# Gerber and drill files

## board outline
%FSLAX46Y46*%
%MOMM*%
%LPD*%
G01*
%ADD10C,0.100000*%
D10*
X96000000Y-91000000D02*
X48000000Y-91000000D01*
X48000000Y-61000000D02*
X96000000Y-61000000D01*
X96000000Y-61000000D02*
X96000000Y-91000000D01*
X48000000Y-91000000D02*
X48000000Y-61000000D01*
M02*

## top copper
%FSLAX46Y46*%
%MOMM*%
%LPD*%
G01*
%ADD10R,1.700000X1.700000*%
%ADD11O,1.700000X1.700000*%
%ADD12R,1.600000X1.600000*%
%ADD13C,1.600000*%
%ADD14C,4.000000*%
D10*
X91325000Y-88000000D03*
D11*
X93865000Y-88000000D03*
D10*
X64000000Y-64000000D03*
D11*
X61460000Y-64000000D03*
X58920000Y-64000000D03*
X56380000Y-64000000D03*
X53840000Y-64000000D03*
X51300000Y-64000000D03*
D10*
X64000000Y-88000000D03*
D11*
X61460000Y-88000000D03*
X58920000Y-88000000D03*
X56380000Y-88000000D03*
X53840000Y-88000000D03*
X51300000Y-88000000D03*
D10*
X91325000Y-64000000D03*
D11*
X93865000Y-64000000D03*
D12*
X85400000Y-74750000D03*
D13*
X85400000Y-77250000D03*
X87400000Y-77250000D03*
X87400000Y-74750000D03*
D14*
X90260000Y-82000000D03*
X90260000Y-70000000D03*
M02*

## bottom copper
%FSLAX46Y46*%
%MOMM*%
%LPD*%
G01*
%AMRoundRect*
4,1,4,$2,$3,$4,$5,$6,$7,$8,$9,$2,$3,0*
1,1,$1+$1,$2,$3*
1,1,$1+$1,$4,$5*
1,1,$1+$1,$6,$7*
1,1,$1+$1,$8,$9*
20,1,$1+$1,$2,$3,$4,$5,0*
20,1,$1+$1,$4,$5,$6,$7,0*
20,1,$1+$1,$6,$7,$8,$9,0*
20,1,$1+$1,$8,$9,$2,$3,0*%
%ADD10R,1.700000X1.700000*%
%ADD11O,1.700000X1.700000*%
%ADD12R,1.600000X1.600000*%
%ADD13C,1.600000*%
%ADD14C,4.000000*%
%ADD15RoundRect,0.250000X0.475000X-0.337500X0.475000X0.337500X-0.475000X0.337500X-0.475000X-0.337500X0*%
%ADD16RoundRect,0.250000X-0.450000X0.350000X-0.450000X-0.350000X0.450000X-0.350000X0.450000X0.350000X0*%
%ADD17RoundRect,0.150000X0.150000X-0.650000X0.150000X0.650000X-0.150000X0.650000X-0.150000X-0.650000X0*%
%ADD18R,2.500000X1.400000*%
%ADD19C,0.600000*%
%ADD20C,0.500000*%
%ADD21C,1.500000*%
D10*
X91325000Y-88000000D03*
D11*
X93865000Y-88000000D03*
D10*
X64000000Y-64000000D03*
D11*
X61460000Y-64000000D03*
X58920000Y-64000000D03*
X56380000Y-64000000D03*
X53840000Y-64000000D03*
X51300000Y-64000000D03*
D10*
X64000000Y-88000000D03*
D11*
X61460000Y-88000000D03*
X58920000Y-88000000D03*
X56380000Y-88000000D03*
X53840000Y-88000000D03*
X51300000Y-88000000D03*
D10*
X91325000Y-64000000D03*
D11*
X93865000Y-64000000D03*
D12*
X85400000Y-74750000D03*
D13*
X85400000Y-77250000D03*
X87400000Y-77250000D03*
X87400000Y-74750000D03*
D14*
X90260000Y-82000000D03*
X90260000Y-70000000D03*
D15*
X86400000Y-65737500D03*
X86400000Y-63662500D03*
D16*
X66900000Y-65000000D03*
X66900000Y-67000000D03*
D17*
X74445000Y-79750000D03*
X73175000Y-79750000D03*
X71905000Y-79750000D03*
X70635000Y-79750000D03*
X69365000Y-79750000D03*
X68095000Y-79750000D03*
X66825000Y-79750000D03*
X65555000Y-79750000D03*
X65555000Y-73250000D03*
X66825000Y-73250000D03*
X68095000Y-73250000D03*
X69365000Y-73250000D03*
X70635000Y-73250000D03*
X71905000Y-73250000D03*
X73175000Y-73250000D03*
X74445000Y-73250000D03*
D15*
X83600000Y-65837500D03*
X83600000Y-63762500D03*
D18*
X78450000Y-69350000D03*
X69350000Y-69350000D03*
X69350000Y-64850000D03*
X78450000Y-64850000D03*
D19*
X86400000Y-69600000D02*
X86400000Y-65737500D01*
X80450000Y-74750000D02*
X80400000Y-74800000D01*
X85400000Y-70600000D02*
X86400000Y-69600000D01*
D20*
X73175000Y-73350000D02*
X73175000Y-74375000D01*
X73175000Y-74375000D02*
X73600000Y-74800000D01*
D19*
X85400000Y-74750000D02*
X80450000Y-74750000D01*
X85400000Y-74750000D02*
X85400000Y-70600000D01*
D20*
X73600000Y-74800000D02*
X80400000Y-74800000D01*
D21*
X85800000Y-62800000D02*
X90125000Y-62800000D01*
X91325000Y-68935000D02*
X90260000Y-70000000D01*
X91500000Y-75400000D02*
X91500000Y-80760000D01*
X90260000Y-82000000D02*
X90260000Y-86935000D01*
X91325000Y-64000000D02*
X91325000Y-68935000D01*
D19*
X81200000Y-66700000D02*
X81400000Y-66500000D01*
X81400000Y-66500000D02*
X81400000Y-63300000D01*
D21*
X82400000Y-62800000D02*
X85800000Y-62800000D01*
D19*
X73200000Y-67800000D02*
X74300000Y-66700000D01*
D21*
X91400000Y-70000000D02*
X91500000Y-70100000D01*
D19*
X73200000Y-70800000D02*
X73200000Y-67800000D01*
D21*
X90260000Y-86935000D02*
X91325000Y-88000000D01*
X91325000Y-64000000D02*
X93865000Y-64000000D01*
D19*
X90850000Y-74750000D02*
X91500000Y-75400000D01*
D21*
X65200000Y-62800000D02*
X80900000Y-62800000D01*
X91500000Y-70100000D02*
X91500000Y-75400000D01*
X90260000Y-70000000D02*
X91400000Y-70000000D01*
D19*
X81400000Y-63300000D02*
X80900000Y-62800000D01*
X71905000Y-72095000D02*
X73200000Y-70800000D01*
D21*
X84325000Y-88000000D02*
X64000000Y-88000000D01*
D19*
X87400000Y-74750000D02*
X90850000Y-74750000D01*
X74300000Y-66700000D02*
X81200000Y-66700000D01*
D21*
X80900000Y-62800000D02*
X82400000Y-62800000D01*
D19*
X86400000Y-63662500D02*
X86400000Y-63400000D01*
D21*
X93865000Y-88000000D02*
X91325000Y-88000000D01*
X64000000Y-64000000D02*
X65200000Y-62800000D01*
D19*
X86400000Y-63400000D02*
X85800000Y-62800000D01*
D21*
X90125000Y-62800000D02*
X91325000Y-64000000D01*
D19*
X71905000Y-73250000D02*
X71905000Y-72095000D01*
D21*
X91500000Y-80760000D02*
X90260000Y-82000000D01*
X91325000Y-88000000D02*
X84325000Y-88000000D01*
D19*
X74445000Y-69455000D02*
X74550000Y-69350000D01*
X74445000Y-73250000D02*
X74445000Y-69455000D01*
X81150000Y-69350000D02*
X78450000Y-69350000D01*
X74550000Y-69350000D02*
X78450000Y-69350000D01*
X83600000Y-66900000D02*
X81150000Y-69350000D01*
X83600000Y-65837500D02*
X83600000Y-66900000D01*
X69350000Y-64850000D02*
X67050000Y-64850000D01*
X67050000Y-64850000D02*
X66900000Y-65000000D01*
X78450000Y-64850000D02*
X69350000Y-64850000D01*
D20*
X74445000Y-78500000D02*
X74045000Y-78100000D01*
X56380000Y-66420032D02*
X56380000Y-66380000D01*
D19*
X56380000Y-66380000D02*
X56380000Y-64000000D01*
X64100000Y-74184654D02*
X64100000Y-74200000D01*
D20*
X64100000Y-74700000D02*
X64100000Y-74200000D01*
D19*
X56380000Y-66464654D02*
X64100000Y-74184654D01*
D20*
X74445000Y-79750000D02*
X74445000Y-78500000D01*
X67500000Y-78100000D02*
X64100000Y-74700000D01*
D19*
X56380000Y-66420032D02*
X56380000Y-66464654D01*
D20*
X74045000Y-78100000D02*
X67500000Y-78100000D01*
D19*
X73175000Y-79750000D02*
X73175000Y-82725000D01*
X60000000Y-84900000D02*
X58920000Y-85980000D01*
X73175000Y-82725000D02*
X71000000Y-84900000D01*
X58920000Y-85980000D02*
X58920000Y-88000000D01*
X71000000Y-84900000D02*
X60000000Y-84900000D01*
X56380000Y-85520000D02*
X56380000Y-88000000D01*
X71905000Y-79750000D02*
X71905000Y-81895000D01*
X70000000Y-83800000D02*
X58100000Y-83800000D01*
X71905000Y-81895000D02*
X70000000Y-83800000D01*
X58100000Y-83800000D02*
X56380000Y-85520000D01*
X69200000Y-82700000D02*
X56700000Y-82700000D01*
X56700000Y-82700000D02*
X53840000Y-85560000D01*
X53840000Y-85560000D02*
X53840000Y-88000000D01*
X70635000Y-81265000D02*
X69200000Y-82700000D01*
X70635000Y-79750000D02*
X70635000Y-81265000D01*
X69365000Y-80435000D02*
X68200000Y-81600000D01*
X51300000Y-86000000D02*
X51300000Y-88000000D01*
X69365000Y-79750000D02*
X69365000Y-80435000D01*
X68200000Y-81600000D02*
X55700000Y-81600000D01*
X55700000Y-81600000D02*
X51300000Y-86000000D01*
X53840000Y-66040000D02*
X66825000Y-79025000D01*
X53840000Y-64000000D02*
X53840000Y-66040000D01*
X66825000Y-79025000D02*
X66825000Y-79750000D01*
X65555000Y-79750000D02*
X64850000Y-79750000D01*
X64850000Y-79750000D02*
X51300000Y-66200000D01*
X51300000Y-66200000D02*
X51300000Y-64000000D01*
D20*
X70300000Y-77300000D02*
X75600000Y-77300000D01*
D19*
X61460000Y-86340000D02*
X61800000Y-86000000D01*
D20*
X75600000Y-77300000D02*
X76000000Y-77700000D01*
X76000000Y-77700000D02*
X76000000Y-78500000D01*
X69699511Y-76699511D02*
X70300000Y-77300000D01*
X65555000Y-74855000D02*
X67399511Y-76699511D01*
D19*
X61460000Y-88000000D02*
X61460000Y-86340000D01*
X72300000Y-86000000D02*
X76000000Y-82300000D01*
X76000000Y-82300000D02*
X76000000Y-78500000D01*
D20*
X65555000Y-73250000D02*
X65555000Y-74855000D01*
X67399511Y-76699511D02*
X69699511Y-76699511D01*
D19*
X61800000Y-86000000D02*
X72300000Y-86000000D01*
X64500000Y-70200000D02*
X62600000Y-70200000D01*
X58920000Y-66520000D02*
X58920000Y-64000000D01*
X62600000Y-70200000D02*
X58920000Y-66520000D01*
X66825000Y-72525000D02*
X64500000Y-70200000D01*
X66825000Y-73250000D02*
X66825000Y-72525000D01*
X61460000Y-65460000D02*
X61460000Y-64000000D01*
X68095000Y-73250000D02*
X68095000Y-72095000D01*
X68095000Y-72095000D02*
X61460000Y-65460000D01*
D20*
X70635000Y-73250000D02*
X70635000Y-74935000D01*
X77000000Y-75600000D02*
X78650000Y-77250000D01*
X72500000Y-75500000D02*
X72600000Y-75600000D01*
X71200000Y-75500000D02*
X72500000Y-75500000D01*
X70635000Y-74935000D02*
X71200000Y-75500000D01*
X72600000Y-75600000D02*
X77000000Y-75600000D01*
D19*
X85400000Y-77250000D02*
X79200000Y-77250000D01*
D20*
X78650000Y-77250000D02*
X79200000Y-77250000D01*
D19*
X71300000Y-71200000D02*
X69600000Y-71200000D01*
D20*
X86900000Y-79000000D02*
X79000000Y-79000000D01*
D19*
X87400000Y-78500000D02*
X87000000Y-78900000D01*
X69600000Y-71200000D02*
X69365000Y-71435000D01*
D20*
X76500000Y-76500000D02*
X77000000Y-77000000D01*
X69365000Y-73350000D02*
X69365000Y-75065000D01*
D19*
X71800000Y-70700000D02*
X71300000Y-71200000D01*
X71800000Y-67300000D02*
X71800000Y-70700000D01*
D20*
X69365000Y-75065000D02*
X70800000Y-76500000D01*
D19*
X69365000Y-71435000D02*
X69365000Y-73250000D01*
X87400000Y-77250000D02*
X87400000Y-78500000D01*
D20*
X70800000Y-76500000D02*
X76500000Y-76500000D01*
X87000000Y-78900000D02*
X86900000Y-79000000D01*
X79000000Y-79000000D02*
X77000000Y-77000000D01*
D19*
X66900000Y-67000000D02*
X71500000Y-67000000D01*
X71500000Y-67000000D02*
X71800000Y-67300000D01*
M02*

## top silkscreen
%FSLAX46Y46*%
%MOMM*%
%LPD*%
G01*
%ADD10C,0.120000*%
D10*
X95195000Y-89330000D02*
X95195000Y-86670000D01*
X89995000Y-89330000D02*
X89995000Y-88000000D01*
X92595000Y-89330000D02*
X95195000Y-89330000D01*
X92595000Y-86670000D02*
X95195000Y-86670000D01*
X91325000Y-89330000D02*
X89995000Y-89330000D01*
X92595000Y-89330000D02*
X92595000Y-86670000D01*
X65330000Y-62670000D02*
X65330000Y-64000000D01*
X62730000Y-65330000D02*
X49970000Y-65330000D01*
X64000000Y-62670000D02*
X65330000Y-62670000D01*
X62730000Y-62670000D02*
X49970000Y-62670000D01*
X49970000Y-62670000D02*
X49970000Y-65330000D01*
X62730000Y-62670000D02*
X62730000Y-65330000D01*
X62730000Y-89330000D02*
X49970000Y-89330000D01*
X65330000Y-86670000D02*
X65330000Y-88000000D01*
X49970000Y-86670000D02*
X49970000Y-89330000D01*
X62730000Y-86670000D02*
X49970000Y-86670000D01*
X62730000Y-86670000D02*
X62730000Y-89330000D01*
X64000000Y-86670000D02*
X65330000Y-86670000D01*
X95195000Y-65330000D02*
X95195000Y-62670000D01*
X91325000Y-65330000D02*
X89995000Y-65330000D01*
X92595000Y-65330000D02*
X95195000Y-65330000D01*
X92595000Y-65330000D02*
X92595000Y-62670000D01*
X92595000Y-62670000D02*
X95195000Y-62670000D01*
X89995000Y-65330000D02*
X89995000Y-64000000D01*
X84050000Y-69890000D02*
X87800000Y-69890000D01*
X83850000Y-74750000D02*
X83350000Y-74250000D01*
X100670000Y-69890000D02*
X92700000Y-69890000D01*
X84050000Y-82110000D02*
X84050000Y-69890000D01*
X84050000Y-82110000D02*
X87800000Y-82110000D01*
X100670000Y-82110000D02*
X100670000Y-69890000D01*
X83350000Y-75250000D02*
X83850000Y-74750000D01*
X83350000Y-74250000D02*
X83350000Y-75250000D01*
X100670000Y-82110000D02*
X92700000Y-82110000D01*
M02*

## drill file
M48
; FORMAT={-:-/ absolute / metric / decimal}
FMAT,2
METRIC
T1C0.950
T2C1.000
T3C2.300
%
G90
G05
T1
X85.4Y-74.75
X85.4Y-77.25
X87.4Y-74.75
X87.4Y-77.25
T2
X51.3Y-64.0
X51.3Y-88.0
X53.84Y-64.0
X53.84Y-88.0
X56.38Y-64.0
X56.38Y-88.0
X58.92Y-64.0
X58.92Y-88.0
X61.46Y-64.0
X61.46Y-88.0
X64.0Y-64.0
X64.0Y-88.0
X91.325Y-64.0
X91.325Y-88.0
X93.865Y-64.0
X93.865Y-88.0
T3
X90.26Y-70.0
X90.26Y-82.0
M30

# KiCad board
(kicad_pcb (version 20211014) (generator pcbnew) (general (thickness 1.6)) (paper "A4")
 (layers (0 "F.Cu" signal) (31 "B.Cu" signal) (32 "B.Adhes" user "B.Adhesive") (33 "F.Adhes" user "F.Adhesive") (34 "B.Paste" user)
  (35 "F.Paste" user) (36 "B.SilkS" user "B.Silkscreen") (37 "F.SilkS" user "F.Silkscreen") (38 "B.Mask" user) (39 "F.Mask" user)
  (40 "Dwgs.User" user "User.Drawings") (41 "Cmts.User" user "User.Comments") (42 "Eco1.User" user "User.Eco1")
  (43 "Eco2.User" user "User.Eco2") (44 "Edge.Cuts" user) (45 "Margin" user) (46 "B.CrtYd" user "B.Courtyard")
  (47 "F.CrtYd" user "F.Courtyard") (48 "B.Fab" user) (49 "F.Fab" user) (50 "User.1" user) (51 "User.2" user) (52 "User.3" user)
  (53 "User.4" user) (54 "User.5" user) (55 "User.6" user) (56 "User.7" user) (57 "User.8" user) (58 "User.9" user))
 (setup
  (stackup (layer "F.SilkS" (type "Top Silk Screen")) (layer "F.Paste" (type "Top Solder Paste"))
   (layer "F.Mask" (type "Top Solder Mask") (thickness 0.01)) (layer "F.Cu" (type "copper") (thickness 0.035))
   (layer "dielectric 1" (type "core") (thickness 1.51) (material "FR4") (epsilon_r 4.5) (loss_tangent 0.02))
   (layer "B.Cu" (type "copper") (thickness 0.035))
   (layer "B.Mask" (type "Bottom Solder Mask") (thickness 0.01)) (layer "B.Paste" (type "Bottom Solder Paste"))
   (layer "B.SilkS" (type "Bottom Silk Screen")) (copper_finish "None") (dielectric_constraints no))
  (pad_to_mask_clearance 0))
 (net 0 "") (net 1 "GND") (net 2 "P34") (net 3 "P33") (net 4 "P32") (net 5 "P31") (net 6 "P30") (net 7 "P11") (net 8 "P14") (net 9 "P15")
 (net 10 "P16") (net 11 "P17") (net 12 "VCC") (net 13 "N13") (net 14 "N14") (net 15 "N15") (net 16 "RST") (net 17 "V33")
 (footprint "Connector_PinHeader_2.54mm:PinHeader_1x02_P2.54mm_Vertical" (layer "F.Cu") (at 91.325 88 90)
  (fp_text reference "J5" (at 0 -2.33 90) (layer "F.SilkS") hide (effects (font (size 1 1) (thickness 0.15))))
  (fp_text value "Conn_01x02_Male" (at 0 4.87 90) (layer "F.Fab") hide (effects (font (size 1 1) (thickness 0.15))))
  (fp_line (start -1.33 3.87) (end 1.33 3.87) (layer "F.SilkS") (width 0.12))
  (fp_line (start -1.33 -1.33) (end 0 -1.33) (layer "F.SilkS") (width 0.12))
  (fp_line (start -1.33 1.27) (end -1.33 3.87) (layer "F.SilkS") (width 0.12))
  (fp_line (start 1.33 1.27) (end 1.33 3.87) (layer "F.SilkS") (width 0.12))
  (fp_line (start -1.33 0) (end -1.33 -1.33) (layer "F.SilkS") (width 0.12))
  (fp_line (start -1.33 1.27) (end 1.33 1.27) (layer "F.SilkS") (width 0.12))
  (pad "1" thru_hole rect locked (at 0 0 90) (size 1.7 1.7) (drill 1) (layers *.Cu *.Mask) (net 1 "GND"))
  (pad "2" thru_hole oval locked (at 0 2.54 90) (size 1.7 1.7) (drill 1) (layers *.Cu *.Mask) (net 1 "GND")))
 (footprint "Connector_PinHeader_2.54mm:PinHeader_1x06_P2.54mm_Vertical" (layer "F.Cu") (at 64 64 -90)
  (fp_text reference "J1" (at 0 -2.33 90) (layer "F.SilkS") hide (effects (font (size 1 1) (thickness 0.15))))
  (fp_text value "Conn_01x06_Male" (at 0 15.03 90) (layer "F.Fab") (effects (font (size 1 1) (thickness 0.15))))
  (fp_line (start -1.33 -1.33) (end 0 -1.33) (layer "F.SilkS") (width 0.12))
  (fp_line (start 1.33 1.27) (end 1.33 14.03) (layer "F.SilkS") (width 0.12))
  (fp_line (start -1.33 0) (end -1.33 -1.33) (layer "F.SilkS") (width 0.12))
  (fp_line (start -1.33 1.27) (end -1.33 14.03) (layer "F.SilkS") (width 0.12))
  (fp_line (start -1.33 14.03) (end 1.33 14.03) (layer "F.SilkS") (width 0.12))
  (fp_line (start -1.33 1.27) (end 1.33 1.27) (layer "F.SilkS") (width 0.12))
  (pad "1" thru_hole rect locked (at 0 0 270) (size 1.7 1.7) (drill 1) (layers *.Cu *.Mask) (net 1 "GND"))
  (pad "2" thru_hole oval locked (at 0 2.54 270) (size 1.7 1.7) (drill 1) (layers *.Cu *.Mask) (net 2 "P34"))
  (pad "3" thru_hole oval locked (at 0 5.08 270) (size 1.7 1.7) (drill 1) (layers *.Cu *.Mask) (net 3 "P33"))
  (pad "4" thru_hole oval locked (at 0 7.62 270) (size 1.7 1.7) (drill 1) (layers *.Cu *.Mask) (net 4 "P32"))
  (pad "5" thru_hole oval locked (at 0 10.16 270) (size 1.7 1.7) (drill 1) (layers *.Cu *.Mask) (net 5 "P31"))
  (pad "6" thru_hole oval locked (at 0 12.7 270) (size 1.7 1.7) (drill 1) (layers *.Cu *.Mask) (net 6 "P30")))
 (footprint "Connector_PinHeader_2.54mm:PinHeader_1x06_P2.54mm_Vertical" (layer "F.Cu") (at 64 88 -90)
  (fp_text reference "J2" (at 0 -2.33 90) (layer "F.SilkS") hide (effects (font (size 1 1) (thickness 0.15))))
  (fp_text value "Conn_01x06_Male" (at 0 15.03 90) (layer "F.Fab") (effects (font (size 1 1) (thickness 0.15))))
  (fp_line (start 1.33 1.27) (end 1.33 14.03) (layer "F.SilkS") (width 0.12))
  (fp_line (start -1.33 -1.33) (end 0 -1.33) (layer "F.SilkS") (width 0.12))
  (fp_line (start -1.33 14.03) (end 1.33 14.03) (layer "F.SilkS") (width 0.12))
  (fp_line (start -1.33 1.27) (end -1.33 14.03) (layer "F.SilkS") (width 0.12))
  (fp_line (start -1.33 1.27) (end 1.33 1.27) (layer "F.SilkS") (width 0.12))
  (fp_line (start -1.33 0) (end -1.33 -1.33) (layer "F.SilkS") (width 0.12))
  (pad "1" thru_hole rect locked (at 0 0 270) (size 1.7 1.7) (drill 1) (layers *.Cu *.Mask) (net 1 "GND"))
  (pad "2" thru_hole oval locked (at 0 2.54 270) (size 1.7 1.7) (drill 1) (layers *.Cu *.Mask) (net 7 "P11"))
  (pad "3" thru_hole oval locked (at 0 5.08 270) (size 1.7 1.7) (drill 1) (layers *.Cu *.Mask) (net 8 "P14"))
  (pad "4" thru_hole oval locked (at 0 7.62 270) (size 1.7 1.7) (drill 1) (layers *.Cu *.Mask) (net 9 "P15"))
  (pad "5" thru_hole oval locked (at 0 10.16 270) (size 1.7 1.7) (drill 1) (layers *.Cu *.Mask) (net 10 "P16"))
  (pad "6" thru_hole oval locked (at 0 12.7 270) (size 1.7 1.7) (drill 1) (layers *.Cu *.Mask) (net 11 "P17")))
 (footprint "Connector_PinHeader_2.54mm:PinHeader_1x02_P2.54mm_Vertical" (layer "F.Cu") (at 91.325 64 90)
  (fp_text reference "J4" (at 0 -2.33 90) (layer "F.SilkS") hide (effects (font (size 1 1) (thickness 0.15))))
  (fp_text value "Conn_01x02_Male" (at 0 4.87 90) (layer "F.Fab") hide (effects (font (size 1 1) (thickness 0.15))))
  (fp_line (start -1.33 3.87) (end 1.33 3.87) (layer "F.SilkS") (width 0.12))
  (fp_line (start -1.33 0) (end -1.33 -1.33) (layer "F.SilkS") (width 0.12))
  (fp_line (start -1.33 1.27) (end -1.33 3.87) (layer "F.SilkS") (width 0.12))
  (fp_line (start -1.33 1.27) (end 1.33 1.27) (layer "F.SilkS") (width 0.12))
  (fp_line (start 1.33 1.27) (end 1.33 3.87) (layer "F.SilkS") (width 0.12))
  (fp_line (start -1.33 -1.33) (end 0 -1.33) (layer "F.SilkS") (width 0.12))
  (pad "1" thru_hole rect locked (at 0 0 90) (size 1.7 1.7) (drill 1) (layers *.Cu *.Mask) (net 1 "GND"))
  (pad "2" thru_hole oval locked (at 0 2.54 90) (size 1.7 1.7) (drill 1) (layers *.Cu *.Mask) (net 1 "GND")))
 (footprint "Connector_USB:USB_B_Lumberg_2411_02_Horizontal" (layer "F.Cu") (at 85.4 74.75)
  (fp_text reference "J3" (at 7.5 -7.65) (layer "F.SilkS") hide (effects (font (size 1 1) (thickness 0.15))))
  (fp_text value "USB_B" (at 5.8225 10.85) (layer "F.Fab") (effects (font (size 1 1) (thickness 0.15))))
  (fp_line (start -1.35 -4.86) (end 2.4 -4.86) (layer "F.SilkS") (width 0.12))
  (fp_line (start -1.55 0) (end -2.05 -0.5) (layer "F.SilkS") (width 0.12))
  (fp_line (start 15.27 -4.86) (end 7.3 -4.86) (layer "F.SilkS") (width 0.12))
  (fp_line (start -1.35 7.36) (end -1.35 -4.86) (layer "F.SilkS") (width 0.12))
  (fp_line (start -1.35 7.36) (end 2.4 7.36) (layer "F.SilkS") (width 0.12))
  (fp_line (start 15.27 7.36) (end 15.27 -4.86) (layer "F.SilkS") (width 0.12))
  (fp_line (start -2.05 0.5) (end -1.55 0) (layer "F.SilkS") (width 0.12))
  (fp_line (start -2.05 -0.5) (end -2.05 0.5) (layer "F.SilkS") (width 0.12))
  (fp_line (start 15.27 7.36) (end 7.3 7.36) (layer "F.SilkS") (width 0.12))
  (pad "1" thru_hole rect locked (at 0 0 90) (size 1.6 1.6) (drill 0.95) (layers *.Cu *.Mask) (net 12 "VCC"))
  (pad "2" thru_hole circle locked (at 0 2.5 90) (size 1.6 1.6) (drill 0.95) (layers *.Cu *.Mask) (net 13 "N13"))
  (pad "3" thru_hole circle locked (at 2 2.5 90) (size 1.6 1.6) (drill 0.95) (layers *.Cu *.Mask) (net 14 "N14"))
  (pad "4" thru_hole circle locked (at 2 0 90) (size 1.6 1.6) (drill 0.95) (layers *.Cu *.Mask) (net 1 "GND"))
  (pad "5" thru_hole circle locked (at 4.86 7.25 90) (size 4 4) (drill 2.3) (layers *.Cu *.Mask) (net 1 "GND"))
  (pad "5" thru_hole circle locked (at 4.86 -4.75 90) (size 4 4) (drill 2.3) (layers *.Cu *.Mask) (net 1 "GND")))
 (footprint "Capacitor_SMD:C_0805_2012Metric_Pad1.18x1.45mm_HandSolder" (layer "B.Cu") (at 86.4 64.7 90)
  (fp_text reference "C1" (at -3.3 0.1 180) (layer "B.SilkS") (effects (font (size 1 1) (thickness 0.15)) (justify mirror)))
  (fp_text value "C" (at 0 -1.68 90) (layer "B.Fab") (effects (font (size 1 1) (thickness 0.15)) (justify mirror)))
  (pad "1" smd roundrect locked (at -1.0375 0 90) (size 1.175 1.45) (layers "B.Cu" "B.Paste" "B.Mask") (roundrect_rratio 0.212766)
   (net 12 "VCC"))
  (pad "2" smd roundrect locked (at 1.0375 0 90) (size 1.175 1.45) (layers "B.Cu" "B.Paste" "B.Mask") (roundrect_rratio 0.212766)
   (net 1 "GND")))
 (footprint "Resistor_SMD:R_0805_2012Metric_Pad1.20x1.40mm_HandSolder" (layer "B.Cu") (at 66.9 66 -90)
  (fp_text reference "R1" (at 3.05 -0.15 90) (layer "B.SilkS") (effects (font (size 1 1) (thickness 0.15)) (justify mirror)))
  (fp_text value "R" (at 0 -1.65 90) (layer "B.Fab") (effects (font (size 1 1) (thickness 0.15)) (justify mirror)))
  (pad "1" smd roundrect locked (at -1 0 270) (size 1.2 1.4) (layers "B.Cu" "B.Paste" "B.Mask") (roundrect_rratio 0.208333) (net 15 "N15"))
  (pad "2" smd roundrect locked (at 1 0 270) (size 1.2 1.4) (layers "B.Cu" "B.Paste" "B.Mask") (roundrect_rratio 0.208333) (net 14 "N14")))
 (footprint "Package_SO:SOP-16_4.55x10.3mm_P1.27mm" (layer "B.Cu") (at 70 76.5 90)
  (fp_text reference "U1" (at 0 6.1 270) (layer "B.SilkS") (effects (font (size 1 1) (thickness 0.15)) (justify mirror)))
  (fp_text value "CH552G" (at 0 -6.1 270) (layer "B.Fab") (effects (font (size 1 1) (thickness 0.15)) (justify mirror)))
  (pad "1" smd roundrect locked (at -3.25 4.445 90) (size 1.6 0.6) (layers "B.Cu" "B.Paste" "B.Mask") (roundrect_rratio 0.25) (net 4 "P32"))
  (pad "2" smd roundrect locked (at -3.25 3.175 90) (size 1.6 0.6) (layers "B.Cu" "B.Paste" "B.Mask") (roundrect_rratio 0.25) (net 8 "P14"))
  (pad "3" smd roundrect locked (at -3.25 1.905 90) (size 1.6 0.6) (layers "B.Cu" "B.Paste" "B.Mask") (roundrect_rratio 0.25) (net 9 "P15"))
  (pad "4" smd roundrect locked (at -3.25 0.635 90) (size 1.6 0.6) (layers "B.Cu" "B.Paste" "B.Mask") (roundrect_rratio 0.25) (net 10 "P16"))
  (pad "5" smd roundrect locked (at -3.25 -0.635 90) (size 1.6 0.6) (layers "B.Cu" "B.Paste" "B.Mask") (roundrect_rratio 0.25)
   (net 11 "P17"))
  (pad "6" smd roundrect locked (at -3.25 -1.905 90) (size 1.6 0.6) (layers "B.Cu" "B.Paste" "B.Mask") (roundrect_rratio 0.25)
   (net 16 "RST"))
  (pad "7" smd roundrect locked (at -3.25 -3.175 90) (size 1.6 0.6) (layers "B.Cu" "B.Paste" "B.Mask") (roundrect_rratio 0.25) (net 5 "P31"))
  (pad "8" smd roundrect locked (at -3.25 -4.445 90) (size 1.6 0.6) (layers "B.Cu" "B.Paste" "B.Mask") (roundrect_rratio 0.25) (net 6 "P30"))
  (pad "9" smd roundrect locked (at 3.25 -4.445 90) (size 1.6 0.6) (layers "B.Cu" "B.Paste" "B.Mask") (roundrect_rratio 0.25) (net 7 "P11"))
  (pad "10" smd roundrect locked (at 3.25 -3.175 90) (size 1.6 0.6) (layers "B.Cu" "B.Paste" "B.Mask") (roundrect_rratio 0.25) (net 3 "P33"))
  (pad "11" smd roundrect locked (at 3.25 -1.905 90) (size 1.6 0.6) (layers "B.Cu" "B.Paste" "B.Mask") (roundrect_rratio 0.25) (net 2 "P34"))
  (pad "12" smd roundrect locked (at 3.25 -0.635 90) (size 1.6 0.6) (layers "B.Cu" "B.Paste" "B.Mask") (roundrect_rratio 0.25)
   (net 14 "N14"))
  (pad "13" smd roundrect locked (at 3.25 0.635 90) (size 1.6 0.6) (layers "B.Cu" "B.Paste" "B.Mask") (roundrect_rratio 0.25) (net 13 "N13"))
  (pad "14" smd roundrect locked (at 3.25 1.905 90) (size 1.6 0.6) (layers "B.Cu" "B.Paste" "B.Mask") (roundrect_rratio 0.25) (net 1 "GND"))
  (pad "15" smd roundrect locked (at 3.25 3.175 90) (size 1.6 0.6) (layers "B.Cu" "B.Paste" "B.Mask") (roundrect_rratio 0.25) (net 12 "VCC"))
  (pad "16" smd roundrect locked (at 3.25 4.445 90) (size 1.6 0.6) (layers "B.Cu" "B.Paste" "B.Mask") (roundrect_rratio 0.25) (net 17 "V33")))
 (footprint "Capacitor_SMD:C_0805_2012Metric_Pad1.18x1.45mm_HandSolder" (layer "B.Cu") (at 83.6 64.8 90)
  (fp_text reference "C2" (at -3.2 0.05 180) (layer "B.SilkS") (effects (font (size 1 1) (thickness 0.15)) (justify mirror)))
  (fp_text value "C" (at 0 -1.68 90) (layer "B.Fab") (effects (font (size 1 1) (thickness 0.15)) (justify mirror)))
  (pad "1" smd roundrect locked (at -1.0375 0 90) (size 1.175 1.45) (layers "B.Cu" "B.Paste" "B.Mask") (roundrect_rratio 0.212766)
   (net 17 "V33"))
  (pad "2" smd roundrect locked (at 1.0375 0 90) (size 1.175 1.45) (layers "B.Cu" "B.Paste" "B.Mask") (roundrect_rratio 0.212766)
   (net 1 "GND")))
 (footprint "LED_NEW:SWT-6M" (layer "B.Cu") (at 73.9 67.1)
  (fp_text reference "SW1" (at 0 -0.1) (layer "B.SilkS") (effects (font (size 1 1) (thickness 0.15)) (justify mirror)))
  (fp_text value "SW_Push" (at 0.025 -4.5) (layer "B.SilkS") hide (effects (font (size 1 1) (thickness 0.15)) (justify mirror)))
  (pad "1" smd rect locked (at 4.55 2.25) (size 2.5 1.4) (layers "B.Cu" "B.Paste" "B.Mask") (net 17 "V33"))
  (pad "1" smd rect locked (at -4.55 2.25) (size 2.5 1.4) (layers "B.Cu" "B.Paste" "B.Mask") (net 17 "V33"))
  (pad "2" smd rect locked (at -4.55 -2.25) (size 2.5 1.4) (layers "B.Cu" "B.Paste" "B.Mask") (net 15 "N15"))
  (pad "2" smd rect locked (at 4.55 -2.25) (size 2.5 1.4) (layers "B.Cu" "B.Paste" "B.Mask") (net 15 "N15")))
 (gr_line (start 96 91) (end 48 91) (layer "Edge.Cuts") (width 0.1))
 (gr_line (start 48 61) (end 96 61) (layer "Edge.Cuts") (width 0.1))
 (gr_line (start 96 61) (end 96 91) (layer "Edge.Cuts") (width 0.1))
 (gr_line (start 48 91) (end 48 61) (layer "Edge.Cuts") (width 0.1))
 (segment (start 86.4 69.6) (end 86.4 65.7375) (width 0.6) (layer "B.Cu") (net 12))
 (segment (start 80.45 74.75) (end 80.4 74.8) (width 0.6) (layer "B.Cu") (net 12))
 (segment (start 85.4 70.6) (end 86.4 69.6) (width 0.6) (layer "B.Cu") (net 12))
 (segment (start 73.175 73.35) (end 73.175 74.375) (width 0.5) (layer "B.Cu") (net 12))
 (segment (start 73.175 74.375) (end 73.6 74.8) (width 0.5) (layer "B.Cu") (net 12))
 (segment (start 85.4 74.75) (end 80.45 74.75) (width 0.6) (layer "B.Cu") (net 12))
 (segment (start 85.4 74.75) (end 85.4 70.6) (width 0.6) (layer "B.Cu") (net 12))
 (segment (start 73.6 74.8) (end 80.4 74.8) (width 0.5) (layer "B.Cu") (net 12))
 (segment (start 85.8 62.8) (end 90.125 62.8) (width 1.5) (layer "B.Cu") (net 1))
 (segment (start 91.325 68.935) (end 90.26 70) (width 1.5) (layer "B.Cu") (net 1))
 (segment (start 91.5 75.4) (end 91.5 80.76) (width 1.5) (layer "B.Cu") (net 1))
 (segment (start 90.26 82) (end 90.26 86.935) (width 1.5) (layer "B.Cu") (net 1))
 (segment (start 91.325 64) (end 91.325 68.935) (width 1.5) (layer "B.Cu") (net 1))
 (segment (start 81.2 66.7) (end 81.4 66.5) (width 0.6) (layer "B.Cu") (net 1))
 (segment (start 81.4 66.5) (end 81.4 63.3) (width 0.6) (layer "B.Cu") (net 1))
 (segment (start 82.4 62.8) (end 85.8 62.8) (width 1.5) (layer "B.Cu") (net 1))
 (segment (start 73.2 67.8) (end 74.3 66.7) (width 0.6) (layer "B.Cu") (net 1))
 (segment (start 91.4 70) (end 91.5 70.1) (width 1.5) (layer "B.Cu") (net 1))
 (segment (start 73.2 70.8) (end 73.2 67.8) (width 0.6) (layer "B.Cu") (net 1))
 (segment (start 90.26 86.935) (end 91.325 88) (width 1.5) (layer "B.Cu") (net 1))
 (segment (start 91.325 64) (end 93.865 64) (width 1.5) (layer "B.Cu") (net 1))
 (segment (start 90.85 74.75) (end 91.5 75.4) (width 0.6) (layer "B.Cu") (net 1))
 (segment (start 65.2 62.8) (end 80.9 62.8) (width 1.5) (layer "B.Cu") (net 1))
 (segment (start 91.5 70.1) (end 91.5 75.4) (width 1.5) (layer "B.Cu") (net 1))
 (segment (start 90.26 70) (end 91.4 70) (width 1.5) (layer "B.Cu") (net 1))
 (segment (start 81.4 63.3) (end 80.9 62.8) (width 0.6) (layer "B.Cu") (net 1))
 (segment (start 71.905 72.095) (end 73.2 70.8) (width 0.6) (layer "B.Cu") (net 1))
 (segment (start 84.325 88) (end 64 88) (width 1.5) (layer "B.Cu") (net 1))
 (segment (start 87.4 74.75) (end 90.85 74.75) (width 0.6) (layer "B.Cu") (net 1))
 (segment (start 74.3 66.7) (end 81.2 66.7) (width 0.6) (layer "B.Cu") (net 1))
 (segment (start 80.9 62.8) (end 82.4 62.8) (width 1.5) (layer "B.Cu") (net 1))
 (segment (start 86.4 63.6625) (end 86.4 63.4) (width 0.6) (layer "B.Cu") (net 1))
 (segment (start 93.865 88) (end 91.325 88) (width 1.5) (layer "B.Cu") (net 1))
 (segment (start 64 64) (end 65.2 62.8) (width 1.5) (layer "B.Cu") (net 1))
 (segment (start 86.4 63.4) (end 85.8 62.8) (width 0.6) (layer "B.Cu") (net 1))
 (segment (start 90.125 62.8) (end 91.325 64) (width 1.5) (layer "B.Cu") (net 1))
 (segment (start 71.905 73.25) (end 71.905 72.095) (width 0.6) (layer "B.Cu") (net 1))
 (segment (start 91.5 80.76) (end 90.26 82) (width 1.5) (layer "B.Cu") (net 1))
 (segment (start 91.325 88) (end 84.325 88) (width 1.5) (layer "B.Cu") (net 1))
 (segment (start 74.445 69.455) (end 74.55 69.35) (width 0.6) (layer "B.Cu") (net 17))
 (segment (start 74.445 73.25) (end 74.445 69.455) (width 0.6) (layer "B.Cu") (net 17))
 (segment (start 81.15 69.35) (end 78.45 69.35) (width 0.6) (layer "B.Cu") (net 17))
 (segment (start 74.55 69.35) (end 78.45 69.35) (width 0.6) (layer "B.Cu") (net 17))
 (segment (start 83.6 66.9) (end 81.15 69.35) (width 0.6) (layer "B.Cu") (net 17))
 (segment (start 83.6 65.8375) (end 83.6 66.9) (width 0.6) (layer "B.Cu") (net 17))
 (segment (start 69.35 64.85) (end 67.05 64.85) (width 0.6) (layer "B.Cu") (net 15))
 (segment (start 67.05 64.85) (end 66.9 65) (width 0.6) (layer "B.Cu") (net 15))
 (segment (start 78.45 64.85) (end 69.35 64.85) (width 0.6) (layer "B.Cu") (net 15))
 (segment (start 74.445 78.5) (end 74.045 78.1) (width 0.5) (layer "B.Cu") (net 4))
 (segment (start 56.38 66.420032) (end 56.38 66.38) (width 0.5) (layer "B.Cu") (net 4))
 (segment (start 56.38 66.38) (end 56.38 64) (width 0.6) (layer "B.Cu") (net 4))
 (segment (start 64.1 74.184654) (end 64.1 74.2) (width 0.6) (layer "B.Cu") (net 4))
 (segment (start 64.1 74.7) (end 64.1 74.2) (width 0.5) (layer "B.Cu") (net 4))
 (segment (start 56.38 66.464654) (end 64.1 74.184654) (width 0.6) (layer "B.Cu") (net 4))
 (segment (start 74.445 79.75) (end 74.445 78.5) (width 0.5) (layer "B.Cu") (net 4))
 (segment (start 67.5 78.1) (end 64.1 74.7) (width 0.5) (layer "B.Cu") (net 4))
 (segment (start 56.38 66.420032) (end 56.38 66.464654) (width 0.6) (layer "B.Cu") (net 4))
 (segment (start 74.045 78.1) (end 67.5 78.1) (width 0.5) (layer "B.Cu") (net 4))
 (segment (start 73.175 79.75) (end 73.175 82.725) (width 0.6) (layer "B.Cu") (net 8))
 (segment (start 60 84.9) (end 58.92 85.98) (width 0.6) (layer "B.Cu") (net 8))
 (segment (start 73.175 82.725) (end 71 84.9) (width 0.6) (layer "B.Cu") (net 8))
 (segment (start 58.92 85.98) (end 58.92 88) (width 0.6) (layer "B.Cu") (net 8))
 (segment (start 71 84.9) (end 60 84.9) (width 0.6) (layer "B.Cu") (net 8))
 (segment (start 56.38 85.52) (end 56.38 88) (width 0.6) (layer "B.Cu") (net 9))
 (segment (start 71.905 79.75) (end 71.905 81.895) (width 0.6) (layer "B.Cu") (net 9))
 (segment (start 70 83.8) (end 58.1 83.8) (width 0.6) (layer "B.Cu") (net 9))
 (segment (start 71.905 81.895) (end 70 83.8) (width 0.6) (layer "B.Cu") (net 9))
 (segment (start 58.1 83.8) (end 56.38 85.52) (width 0.6) (layer "B.Cu") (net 9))
 (segment (start 69.2 82.7) (end 56.7 82.7) (width 0.6) (layer "B.Cu") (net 10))
 (segment (start 56.7 82.7) (end 53.84 85.56) (width 0.6) (layer "B.Cu") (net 10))
 (segment (start 53.84 85.56) (end 53.84 88) (width 0.6) (layer "B.Cu") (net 10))
 (segment (start 70.635 81.265) (end 69.2 82.7) (width 0.6) (layer "B.Cu") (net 10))
 (segment (start 70.635 79.75) (end 70.635 81.265) (width 0.6) (layer "B.Cu") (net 10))
 (segment (start 69.365 80.435) (end 68.2 81.6) (width 0.6) (layer "B.Cu") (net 11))
 (segment (start 51.3 86) (end 51.3 88) (width 0.6) (layer "B.Cu") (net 11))
 (segment (start 69.365 79.75) (end 69.365 80.435) (width 0.6) (layer "B.Cu") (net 11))
 (segment (start 68.2 81.6) (end 55.7 81.6) (width 0.6) (layer "B.Cu") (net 11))
 (segment (start 55.7 81.6) (end 51.3 86) (width 0.6) (layer "B.Cu") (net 11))
 (segment (start 53.84 66.04) (end 66.825 79.025) (width 0.6) (layer "B.Cu") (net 5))
 (segment (start 53.84 64) (end 53.84 66.04) (width 0.6) (layer "B.Cu") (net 5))
 (segment (start 66.825 79.025) (end 66.825 79.75) (width 0.6) (layer "B.Cu") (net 5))
 (segment (start 65.555 79.75) (end 64.85 79.75) (width 0.6) (layer "B.Cu") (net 6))
 (segment (start 64.85 79.75) (end 51.3 66.2) (width 0.6) (layer "B.Cu") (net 6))
 (segment (start 51.3 66.2) (end 51.3 64) (width 0.6) (layer "B.Cu") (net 6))
 (segment (start 70.3 77.3) (end 75.6 77.3) (width 0.5) (layer "B.Cu") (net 7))
 (segment (start 61.46 86.34) (end 61.8 86) (width 0.6) (layer "B.Cu") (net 7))
 (segment (start 75.6 77.3) (end 76 77.7) (width 0.5) (layer "B.Cu") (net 7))
 (segment (start 76 77.7) (end 76 78.5) (width 0.5) (layer "B.Cu") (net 7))
 (segment (start 69.699511 76.699511) (end 70.3 77.3) (width 0.5) (layer "B.Cu") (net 7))
 (segment (start 65.555 74.855) (end 67.399511 76.699511) (width 0.5) (layer "B.Cu") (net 7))
 (segment (start 61.46 88) (end 61.46 86.34) (width 0.6) (layer "B.Cu") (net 7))
 (segment (start 72.3 86) (end 76 82.3) (width 0.6) (layer "B.Cu") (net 7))
 (segment (start 76 82.3) (end 76 78.5) (width 0.6) (layer "B.Cu") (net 7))
 (segment (start 65.555 73.25) (end 65.555 74.855) (width 0.5) (layer "B.Cu") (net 7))
 (segment (start 67.399511 76.699511) (end 69.699511 76.699511) (width 0.5) (layer "B.Cu") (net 7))
 (segment (start 61.8 86) (end 72.3 86) (width 0.6) (layer "B.Cu") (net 7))
 (segment (start 64.5 70.2) (end 62.6 70.2) (width 0.6) (layer "B.Cu") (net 3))
 (segment (start 58.92 66.52) (end 58.92 64) (width 0.6) (layer "B.Cu") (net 3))
 (segment (start 62.6 70.2) (end 58.92 66.52) (width 0.6) (layer "B.Cu") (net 3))
 (segment (start 66.825 72.525) (end 64.5 70.2) (width 0.6) (layer "B.Cu") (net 3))
 (segment (start 66.825 73.25) (end 66.825 72.525) (width 0.6) (layer "B.Cu") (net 3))
 (segment (start 61.46 65.46) (end 61.46 64) (width 0.6) (layer "B.Cu") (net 2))
 (segment (start 68.095 73.25) (end 68.095 72.095) (width 0.6) (layer "B.Cu") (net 2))
 (segment (start 68.095 72.095) (end 61.46 65.46) (width 0.6) (layer "B.Cu") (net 2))
 (segment (start 70.635 73.25) (end 70.635 74.935) (width 0.5) (layer "B.Cu") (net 13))
 (segment (start 77 75.6) (end 78.65 77.25) (width 0.5) (layer "B.Cu") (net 13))
 (segment (start 72.5 75.5) (end 72.6 75.6) (width 0.5) (layer "B.Cu") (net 13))
 (segment (start 71.2 75.5) (end 72.5 75.5) (width 0.5) (layer "B.Cu") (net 13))
 (segment (start 70.635 74.935) (end 71.2 75.5) (width 0.5) (layer "B.Cu") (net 13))
 (segment (start 72.6 75.6) (end 77 75.6) (width 0.5) (layer "B.Cu") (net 13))
 (segment (start 85.4 77.25) (end 79.2 77.25) (width 0.6) (layer "B.Cu") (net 13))
 (segment (start 78.65 77.25) (end 79.2 77.25) (width 0.5) (layer "B.Cu") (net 13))
 (segment (start 71.3 71.2) (end 69.6 71.2) (width 0.6) (layer "B.Cu") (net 14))
 (segment (start 86.9 79) (end 79 79) (width 0.5) (layer "B.Cu") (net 14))
 (segment (start 87.4 78.5) (end 87 78.9) (width 0.6) (layer "B.Cu") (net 14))
 (segment (start 69.6 71.2) (end 69.365 71.435) (width 0.6) (layer "B.Cu") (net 14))
 (segment (start 76.5 76.5) (end 77 77) (width 0.5) (layer "B.Cu") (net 14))
 (segment (start 69.365 73.35) (end 69.365 75.065) (width 0.5) (layer "B.Cu") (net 14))
 (segment (start 71.8 70.7) (end 71.3 71.2) (width 0.6) (layer "B.Cu") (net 14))
 (segment (start 71.8 67.3) (end 71.8 70.7) (width 0.6) (layer "B.Cu") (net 14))
 (segment (start 69.365 75.065) (end 70.8 76.5) (width 0.5) (layer "B.Cu") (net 14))
 (segment (start 69.365 71.435) (end 69.365 73.25) (width 0.6) (layer "B.Cu") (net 14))
 (segment (start 87.4 77.25) (end 87.4 78.5) (width 0.6) (layer "B.Cu") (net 14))
 (segment (start 70.8 76.5) (end 76.5 76.5) (width 0.5) (layer "B.Cu") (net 14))
 (segment (start 87 78.9) (end 86.9 79) (width 0.5) (layer "B.Cu") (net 14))
 (segment (start 79 79) (end 77 77) (width 0.5) (layer "B.Cu") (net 14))
 (segment (start 66.9 67) (end 71.5 67) (width 0.6) (layer "B.Cu") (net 14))
 (segment (start 71.5 67) (end 71.8 67.3) (width 0.6) (layer "B.Cu") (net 14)))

